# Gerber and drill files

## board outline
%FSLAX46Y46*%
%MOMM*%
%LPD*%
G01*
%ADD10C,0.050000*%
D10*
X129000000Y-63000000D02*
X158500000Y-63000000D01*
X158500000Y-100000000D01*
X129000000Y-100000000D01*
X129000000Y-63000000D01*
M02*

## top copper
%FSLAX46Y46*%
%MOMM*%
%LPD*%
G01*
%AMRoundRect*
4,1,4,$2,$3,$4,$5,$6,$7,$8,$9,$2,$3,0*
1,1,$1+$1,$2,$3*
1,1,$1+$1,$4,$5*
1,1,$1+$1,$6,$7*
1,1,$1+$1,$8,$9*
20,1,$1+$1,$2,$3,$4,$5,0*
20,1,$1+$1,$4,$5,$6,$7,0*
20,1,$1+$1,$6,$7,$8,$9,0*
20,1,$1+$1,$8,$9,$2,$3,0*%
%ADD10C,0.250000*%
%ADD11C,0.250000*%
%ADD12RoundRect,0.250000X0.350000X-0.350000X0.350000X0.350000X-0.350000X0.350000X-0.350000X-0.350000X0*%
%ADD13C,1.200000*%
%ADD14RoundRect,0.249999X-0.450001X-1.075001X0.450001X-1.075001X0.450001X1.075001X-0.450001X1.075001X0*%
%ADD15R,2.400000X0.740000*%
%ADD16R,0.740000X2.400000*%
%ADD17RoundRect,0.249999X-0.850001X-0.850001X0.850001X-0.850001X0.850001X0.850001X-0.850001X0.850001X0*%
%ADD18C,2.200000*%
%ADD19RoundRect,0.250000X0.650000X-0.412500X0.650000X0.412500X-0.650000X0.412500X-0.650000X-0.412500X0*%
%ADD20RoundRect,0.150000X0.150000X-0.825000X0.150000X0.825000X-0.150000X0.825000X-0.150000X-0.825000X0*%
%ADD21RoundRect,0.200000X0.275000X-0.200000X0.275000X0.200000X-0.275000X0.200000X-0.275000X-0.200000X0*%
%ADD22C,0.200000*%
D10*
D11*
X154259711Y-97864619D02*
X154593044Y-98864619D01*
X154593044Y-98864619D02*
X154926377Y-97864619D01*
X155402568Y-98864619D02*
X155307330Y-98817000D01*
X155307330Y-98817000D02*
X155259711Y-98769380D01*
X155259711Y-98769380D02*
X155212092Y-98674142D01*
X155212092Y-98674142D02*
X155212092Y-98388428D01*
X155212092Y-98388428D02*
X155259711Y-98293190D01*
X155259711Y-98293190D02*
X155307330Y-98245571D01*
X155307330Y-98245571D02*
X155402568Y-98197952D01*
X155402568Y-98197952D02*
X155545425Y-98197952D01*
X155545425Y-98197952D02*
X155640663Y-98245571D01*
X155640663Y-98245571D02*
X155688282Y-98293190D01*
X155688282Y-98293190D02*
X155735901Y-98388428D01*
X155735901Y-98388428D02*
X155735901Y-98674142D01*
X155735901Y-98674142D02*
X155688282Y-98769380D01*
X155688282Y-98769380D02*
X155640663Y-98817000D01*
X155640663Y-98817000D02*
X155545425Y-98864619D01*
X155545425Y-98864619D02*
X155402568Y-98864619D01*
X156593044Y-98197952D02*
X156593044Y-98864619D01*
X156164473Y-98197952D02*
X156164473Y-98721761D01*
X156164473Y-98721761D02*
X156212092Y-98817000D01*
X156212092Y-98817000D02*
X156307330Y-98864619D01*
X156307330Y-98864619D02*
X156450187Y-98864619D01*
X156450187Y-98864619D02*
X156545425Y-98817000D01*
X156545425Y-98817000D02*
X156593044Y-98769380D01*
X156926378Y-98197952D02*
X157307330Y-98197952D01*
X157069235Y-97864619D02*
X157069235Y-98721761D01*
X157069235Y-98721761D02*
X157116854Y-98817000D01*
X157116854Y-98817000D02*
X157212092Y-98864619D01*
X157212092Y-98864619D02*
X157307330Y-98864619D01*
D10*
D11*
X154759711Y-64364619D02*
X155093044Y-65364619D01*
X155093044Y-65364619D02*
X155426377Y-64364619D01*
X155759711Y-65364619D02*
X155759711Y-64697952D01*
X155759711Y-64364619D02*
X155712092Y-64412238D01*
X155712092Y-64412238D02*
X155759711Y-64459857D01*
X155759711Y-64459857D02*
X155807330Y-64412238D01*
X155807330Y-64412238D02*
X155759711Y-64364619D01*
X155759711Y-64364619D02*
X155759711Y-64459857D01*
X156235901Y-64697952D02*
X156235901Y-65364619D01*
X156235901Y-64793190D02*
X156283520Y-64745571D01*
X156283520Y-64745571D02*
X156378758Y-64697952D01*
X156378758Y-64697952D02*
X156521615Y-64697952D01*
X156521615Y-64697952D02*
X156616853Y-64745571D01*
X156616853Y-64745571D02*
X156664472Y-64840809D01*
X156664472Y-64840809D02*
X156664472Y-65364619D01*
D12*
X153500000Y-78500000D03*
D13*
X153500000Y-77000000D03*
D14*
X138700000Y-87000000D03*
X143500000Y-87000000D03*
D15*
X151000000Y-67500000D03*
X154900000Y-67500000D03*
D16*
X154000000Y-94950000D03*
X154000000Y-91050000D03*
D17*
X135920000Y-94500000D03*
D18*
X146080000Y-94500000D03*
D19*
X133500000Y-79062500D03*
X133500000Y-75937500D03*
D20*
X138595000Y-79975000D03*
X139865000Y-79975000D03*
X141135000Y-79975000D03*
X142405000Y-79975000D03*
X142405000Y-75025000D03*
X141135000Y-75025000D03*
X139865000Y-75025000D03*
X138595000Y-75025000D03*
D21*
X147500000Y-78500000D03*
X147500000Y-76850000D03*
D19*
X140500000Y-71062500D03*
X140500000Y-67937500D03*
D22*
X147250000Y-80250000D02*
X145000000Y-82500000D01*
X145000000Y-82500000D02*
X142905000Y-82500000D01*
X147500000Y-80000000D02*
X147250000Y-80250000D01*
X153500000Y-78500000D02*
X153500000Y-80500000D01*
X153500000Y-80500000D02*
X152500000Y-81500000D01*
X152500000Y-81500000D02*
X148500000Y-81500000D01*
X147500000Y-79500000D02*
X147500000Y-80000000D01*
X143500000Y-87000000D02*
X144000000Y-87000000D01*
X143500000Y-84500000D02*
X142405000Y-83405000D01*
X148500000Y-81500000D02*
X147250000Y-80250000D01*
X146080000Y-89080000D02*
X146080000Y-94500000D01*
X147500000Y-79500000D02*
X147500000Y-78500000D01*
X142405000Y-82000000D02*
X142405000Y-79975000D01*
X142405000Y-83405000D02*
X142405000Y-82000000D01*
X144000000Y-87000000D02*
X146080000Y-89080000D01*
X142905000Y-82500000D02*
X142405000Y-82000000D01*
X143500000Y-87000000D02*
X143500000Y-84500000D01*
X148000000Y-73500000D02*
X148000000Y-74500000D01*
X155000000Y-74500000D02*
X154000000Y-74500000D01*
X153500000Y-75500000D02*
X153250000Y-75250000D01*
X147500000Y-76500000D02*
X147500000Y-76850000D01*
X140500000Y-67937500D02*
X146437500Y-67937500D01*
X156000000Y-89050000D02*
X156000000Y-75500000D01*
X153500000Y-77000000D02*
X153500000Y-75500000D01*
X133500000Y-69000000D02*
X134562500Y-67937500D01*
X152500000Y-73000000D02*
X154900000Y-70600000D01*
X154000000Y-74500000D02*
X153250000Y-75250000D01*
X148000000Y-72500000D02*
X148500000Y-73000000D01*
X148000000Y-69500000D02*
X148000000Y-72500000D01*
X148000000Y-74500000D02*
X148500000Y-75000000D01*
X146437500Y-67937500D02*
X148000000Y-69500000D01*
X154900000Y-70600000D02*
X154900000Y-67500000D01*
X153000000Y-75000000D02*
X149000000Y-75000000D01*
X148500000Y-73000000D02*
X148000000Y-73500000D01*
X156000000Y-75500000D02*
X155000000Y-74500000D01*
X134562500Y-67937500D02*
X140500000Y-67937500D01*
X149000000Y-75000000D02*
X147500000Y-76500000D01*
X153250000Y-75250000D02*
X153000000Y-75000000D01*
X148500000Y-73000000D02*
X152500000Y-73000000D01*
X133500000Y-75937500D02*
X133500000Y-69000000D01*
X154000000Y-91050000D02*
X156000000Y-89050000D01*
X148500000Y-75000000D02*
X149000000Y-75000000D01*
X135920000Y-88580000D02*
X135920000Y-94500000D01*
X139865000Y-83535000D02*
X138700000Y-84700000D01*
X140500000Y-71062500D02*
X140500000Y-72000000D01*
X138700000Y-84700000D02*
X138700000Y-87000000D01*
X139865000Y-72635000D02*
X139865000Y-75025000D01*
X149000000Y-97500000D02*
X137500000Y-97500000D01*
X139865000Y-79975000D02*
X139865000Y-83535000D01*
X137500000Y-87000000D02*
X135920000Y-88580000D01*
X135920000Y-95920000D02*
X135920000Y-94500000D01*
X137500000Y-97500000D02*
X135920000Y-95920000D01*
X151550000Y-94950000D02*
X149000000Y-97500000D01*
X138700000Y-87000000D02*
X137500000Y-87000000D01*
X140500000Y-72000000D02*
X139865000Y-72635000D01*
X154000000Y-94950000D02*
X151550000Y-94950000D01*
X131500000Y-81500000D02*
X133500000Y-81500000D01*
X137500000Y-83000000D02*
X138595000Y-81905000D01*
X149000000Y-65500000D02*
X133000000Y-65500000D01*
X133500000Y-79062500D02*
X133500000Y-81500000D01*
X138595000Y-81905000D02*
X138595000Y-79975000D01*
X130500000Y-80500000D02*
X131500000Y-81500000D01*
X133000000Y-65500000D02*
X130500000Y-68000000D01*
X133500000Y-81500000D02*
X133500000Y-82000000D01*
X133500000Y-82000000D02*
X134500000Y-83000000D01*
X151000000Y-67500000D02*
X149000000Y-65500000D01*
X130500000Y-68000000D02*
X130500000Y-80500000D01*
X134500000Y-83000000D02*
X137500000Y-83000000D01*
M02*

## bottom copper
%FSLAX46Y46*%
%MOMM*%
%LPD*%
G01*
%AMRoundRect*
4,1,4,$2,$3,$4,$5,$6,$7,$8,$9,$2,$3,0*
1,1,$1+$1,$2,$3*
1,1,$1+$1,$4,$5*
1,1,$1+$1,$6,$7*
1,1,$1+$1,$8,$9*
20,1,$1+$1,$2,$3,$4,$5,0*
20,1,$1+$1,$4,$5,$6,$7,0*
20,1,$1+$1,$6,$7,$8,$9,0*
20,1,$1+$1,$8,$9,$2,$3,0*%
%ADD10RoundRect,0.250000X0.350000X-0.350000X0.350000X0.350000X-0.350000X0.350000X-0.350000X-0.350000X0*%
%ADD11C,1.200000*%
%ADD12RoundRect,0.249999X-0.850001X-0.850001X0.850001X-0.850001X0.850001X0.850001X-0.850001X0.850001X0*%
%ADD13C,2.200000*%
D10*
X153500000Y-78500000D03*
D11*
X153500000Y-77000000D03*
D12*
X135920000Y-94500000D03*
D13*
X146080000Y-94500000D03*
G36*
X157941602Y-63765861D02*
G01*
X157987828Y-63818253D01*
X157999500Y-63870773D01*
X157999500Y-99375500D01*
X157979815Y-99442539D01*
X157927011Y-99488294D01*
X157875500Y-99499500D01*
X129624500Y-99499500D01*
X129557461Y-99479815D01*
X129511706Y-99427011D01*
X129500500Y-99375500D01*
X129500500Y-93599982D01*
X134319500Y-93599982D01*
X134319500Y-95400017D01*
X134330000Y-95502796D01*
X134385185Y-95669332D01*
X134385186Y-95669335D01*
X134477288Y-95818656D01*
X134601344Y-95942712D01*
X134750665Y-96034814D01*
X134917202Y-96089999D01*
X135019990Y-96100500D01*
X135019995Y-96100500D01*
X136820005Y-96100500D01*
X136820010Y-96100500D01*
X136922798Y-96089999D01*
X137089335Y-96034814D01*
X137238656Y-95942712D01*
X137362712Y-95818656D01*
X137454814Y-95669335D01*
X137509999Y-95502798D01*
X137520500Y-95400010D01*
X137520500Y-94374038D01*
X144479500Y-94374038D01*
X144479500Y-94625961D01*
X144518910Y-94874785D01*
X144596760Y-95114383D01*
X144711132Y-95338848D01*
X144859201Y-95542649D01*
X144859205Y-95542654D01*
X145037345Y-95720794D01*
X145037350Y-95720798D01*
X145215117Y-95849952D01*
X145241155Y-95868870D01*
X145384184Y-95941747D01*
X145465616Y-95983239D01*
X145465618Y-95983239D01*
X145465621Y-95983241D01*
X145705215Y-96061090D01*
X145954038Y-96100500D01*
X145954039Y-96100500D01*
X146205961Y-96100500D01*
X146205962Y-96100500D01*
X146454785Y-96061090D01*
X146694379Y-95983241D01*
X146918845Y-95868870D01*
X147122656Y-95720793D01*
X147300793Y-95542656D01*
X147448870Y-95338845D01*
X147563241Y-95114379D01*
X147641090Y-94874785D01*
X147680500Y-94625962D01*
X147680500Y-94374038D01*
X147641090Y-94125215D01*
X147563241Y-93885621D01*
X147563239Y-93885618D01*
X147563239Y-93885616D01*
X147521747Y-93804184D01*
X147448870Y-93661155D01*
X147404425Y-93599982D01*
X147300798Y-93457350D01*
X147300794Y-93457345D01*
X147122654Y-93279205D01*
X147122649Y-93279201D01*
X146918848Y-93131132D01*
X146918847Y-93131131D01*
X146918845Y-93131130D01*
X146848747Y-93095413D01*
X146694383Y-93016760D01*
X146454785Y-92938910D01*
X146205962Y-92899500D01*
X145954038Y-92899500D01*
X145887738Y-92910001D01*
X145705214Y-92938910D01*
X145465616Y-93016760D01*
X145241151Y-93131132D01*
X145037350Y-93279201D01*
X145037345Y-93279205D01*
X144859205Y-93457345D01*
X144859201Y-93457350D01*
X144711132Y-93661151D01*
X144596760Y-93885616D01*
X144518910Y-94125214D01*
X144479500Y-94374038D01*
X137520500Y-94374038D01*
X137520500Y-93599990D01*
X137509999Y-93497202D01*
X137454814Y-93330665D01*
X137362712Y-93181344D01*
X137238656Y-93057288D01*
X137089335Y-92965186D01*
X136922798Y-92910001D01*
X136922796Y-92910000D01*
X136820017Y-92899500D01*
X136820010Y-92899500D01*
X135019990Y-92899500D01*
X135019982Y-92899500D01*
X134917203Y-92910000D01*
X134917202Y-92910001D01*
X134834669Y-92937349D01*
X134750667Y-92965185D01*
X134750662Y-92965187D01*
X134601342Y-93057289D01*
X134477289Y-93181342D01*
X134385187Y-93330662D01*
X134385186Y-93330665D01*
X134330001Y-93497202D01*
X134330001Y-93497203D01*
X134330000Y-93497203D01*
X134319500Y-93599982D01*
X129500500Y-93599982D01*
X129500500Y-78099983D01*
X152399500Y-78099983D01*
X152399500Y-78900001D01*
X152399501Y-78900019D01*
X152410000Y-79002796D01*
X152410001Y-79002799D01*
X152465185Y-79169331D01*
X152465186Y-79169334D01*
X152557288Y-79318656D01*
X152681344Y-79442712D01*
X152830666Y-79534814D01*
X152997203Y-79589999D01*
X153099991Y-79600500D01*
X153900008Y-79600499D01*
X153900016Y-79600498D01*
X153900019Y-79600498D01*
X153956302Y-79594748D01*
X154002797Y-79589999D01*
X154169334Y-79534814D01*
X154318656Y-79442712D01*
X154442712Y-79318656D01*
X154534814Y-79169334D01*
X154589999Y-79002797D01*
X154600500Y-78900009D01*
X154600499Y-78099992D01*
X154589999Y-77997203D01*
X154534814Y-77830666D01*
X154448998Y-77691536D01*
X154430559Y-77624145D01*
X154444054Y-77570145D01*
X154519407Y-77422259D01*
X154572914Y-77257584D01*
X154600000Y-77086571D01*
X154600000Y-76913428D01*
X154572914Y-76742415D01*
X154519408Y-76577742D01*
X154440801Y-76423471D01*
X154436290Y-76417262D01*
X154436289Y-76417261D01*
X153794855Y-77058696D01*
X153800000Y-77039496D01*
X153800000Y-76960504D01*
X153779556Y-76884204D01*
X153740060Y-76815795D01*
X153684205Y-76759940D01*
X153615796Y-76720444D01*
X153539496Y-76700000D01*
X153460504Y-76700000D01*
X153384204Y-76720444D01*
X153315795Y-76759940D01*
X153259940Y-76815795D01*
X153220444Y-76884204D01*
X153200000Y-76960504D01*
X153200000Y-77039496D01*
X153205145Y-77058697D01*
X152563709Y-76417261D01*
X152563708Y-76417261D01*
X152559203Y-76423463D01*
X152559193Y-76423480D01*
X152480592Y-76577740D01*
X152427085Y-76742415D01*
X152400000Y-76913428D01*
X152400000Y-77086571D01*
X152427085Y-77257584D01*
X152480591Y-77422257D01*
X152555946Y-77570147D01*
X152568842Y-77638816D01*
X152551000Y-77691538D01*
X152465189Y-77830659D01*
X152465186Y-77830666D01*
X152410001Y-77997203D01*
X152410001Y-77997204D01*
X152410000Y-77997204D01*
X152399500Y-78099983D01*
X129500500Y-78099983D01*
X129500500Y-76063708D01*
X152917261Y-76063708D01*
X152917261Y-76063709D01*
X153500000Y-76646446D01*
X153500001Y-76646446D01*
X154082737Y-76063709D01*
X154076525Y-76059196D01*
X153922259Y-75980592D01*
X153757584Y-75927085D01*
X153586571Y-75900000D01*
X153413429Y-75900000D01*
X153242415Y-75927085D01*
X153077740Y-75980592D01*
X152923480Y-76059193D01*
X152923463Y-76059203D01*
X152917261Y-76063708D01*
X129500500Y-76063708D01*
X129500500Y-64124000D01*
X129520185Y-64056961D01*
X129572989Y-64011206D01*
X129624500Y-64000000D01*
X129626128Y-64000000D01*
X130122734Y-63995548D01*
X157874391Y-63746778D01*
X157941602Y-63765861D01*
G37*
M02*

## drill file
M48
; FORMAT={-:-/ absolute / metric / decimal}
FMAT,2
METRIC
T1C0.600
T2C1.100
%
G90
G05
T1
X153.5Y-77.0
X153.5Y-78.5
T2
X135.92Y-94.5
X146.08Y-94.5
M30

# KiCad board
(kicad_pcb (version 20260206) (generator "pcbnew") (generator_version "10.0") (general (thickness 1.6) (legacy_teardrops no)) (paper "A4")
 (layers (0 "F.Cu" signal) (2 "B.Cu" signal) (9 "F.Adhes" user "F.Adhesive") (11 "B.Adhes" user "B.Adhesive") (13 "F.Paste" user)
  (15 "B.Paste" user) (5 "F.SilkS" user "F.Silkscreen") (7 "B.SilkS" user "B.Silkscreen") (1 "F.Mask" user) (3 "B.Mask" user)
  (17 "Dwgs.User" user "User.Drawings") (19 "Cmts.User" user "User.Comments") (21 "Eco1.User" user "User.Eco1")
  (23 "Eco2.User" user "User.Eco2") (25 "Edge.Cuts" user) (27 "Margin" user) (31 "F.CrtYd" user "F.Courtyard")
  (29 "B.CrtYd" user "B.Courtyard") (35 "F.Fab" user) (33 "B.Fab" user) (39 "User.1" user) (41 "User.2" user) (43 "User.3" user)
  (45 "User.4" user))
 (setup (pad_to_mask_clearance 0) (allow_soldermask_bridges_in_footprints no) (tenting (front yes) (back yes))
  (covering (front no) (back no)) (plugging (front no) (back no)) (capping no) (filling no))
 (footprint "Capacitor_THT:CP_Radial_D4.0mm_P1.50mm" (layer "F.Cu") (at 153.5 78.5 90)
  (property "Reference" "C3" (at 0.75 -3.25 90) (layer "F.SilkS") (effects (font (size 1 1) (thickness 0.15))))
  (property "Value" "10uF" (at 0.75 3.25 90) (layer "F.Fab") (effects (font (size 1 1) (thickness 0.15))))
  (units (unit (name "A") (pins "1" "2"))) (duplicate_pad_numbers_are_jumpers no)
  (pad "1" thru_hole roundrect (at 0 0 90) (size 1.2 1.2) (drill 0.6) (layers "*.Cu" "*.Mask") (remove_unused_layers no)
   (roundrect_rratio 0.208333) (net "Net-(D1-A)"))
  (pad "2" thru_hole circle (at 1.5 0 90) (size 1.2 1.2) (drill 0.6) (layers "*.Cu" "*.Mask") (remove_unused_layers no) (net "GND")))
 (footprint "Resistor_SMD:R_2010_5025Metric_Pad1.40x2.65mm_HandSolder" (layer "F.Cu") (at 141.1 87)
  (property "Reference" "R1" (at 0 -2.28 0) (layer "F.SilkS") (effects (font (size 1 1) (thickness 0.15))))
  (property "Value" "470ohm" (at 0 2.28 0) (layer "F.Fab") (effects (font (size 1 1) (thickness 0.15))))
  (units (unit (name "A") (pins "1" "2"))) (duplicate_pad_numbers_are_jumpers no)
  (pad "1" smd roundrect (at -2.4 0) (size 1.4 2.65) (layers "F.Cu" "F.Mask" "F.Paste") (roundrect_rratio 0.178571) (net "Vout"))
  (pad "2" smd roundrect (at 2.4 0) (size 1.4 2.65) (layers "F.Cu" "F.Mask" "F.Paste") (roundrect_rratio 0.178571) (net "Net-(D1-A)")))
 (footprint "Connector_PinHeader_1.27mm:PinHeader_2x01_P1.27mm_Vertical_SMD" (layer "F.Cu") (at 152.95 67.5)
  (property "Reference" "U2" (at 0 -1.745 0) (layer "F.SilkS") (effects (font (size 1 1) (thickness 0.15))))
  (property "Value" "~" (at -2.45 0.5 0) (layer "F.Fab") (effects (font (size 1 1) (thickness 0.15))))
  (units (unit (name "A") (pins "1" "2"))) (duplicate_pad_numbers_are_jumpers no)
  (pad "1" smd rect (at -1.95 0) (size 2.4 0.74) (layers "F.Cu" "F.Mask" "F.Paste") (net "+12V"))
  (pad "2" smd rect (at 1.95 0) (size 2.4 0.74) (layers "F.Cu" "F.Mask" "F.Paste") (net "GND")))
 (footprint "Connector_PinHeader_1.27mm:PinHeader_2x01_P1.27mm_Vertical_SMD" (layer "F.Cu") (at 154 93 90)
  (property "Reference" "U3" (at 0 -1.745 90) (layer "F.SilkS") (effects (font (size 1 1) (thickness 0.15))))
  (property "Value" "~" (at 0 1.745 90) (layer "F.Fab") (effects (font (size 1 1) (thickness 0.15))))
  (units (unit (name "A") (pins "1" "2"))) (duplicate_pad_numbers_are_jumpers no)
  (pad "1" smd rect (at -1.95 0 90) (size 2.4 0.74) (layers "F.Cu" "F.Mask" "F.Paste") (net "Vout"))
  (pad "2" smd rect (at 1.95 0 90) (size 2.4 0.74) (layers "F.Cu" "F.Mask" "F.Paste") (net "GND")))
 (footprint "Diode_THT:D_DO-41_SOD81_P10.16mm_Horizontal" (layer "F.Cu") (at 135.92 94.5)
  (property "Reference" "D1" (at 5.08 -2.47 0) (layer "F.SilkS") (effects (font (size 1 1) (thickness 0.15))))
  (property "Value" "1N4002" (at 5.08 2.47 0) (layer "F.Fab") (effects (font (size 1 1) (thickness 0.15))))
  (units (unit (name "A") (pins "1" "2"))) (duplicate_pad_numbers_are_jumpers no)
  (pad "1" thru_hole roundrect (at 0 0) (size 2.2 2.2) (drill 1.1) (layers "*.Cu" "*.Mask") (remove_unused_layers no)
   (roundrect_rratio 0.113636) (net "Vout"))
  (pad "2" thru_hole circle (at 10.16 0) (size 2.2 2.2) (drill 1.1) (layers "*.Cu" "*.Mask") (remove_unused_layers no) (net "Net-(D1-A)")))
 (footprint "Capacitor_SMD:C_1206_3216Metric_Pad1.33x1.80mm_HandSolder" (layer "F.Cu") (at 133.5 77.5 90)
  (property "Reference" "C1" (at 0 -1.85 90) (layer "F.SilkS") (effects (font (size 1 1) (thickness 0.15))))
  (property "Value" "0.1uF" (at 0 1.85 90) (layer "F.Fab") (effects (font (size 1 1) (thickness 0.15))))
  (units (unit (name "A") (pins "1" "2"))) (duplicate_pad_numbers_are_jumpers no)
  (pad "1" smd roundrect (at -1.5625 0 90) (size 1.325 1.8) (layers "F.Cu" "F.Mask" "F.Paste") (roundrect_rratio 0.188679) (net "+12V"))
  (pad "2" smd roundrect (at 1.5625 0 90) (size 1.325 1.8) (layers "F.Cu" "F.Mask" "F.Paste") (roundrect_rratio 0.188679) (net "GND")))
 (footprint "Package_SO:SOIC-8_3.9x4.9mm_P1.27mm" (layer "F.Cu") (at 140.5 77.5 90)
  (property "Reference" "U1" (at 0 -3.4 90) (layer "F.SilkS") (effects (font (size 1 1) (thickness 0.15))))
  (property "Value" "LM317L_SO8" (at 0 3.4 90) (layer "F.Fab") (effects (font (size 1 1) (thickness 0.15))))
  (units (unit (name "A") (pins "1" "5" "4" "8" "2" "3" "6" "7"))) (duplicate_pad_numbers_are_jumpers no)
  (pad "1" smd roundrect (at -2.475 -1.905 90) (size 1.95 0.6) (layers "F.Cu" "F.Mask" "F.Paste") (roundrect_rratio 0.25) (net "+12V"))
  (pad "2" smd roundrect (at -2.475 -0.635 90) (size 1.95 0.6) (layers "F.Cu" "F.Mask" "F.Paste") (roundrect_rratio 0.25) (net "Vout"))
  (pad "3" smd roundrect (at -2.475 0.635 90) (size 1.95 0.6) (layers "F.Cu" "F.Mask" "F.Paste") (roundrect_rratio 0.25) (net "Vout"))
  (pad "4" smd roundrect (at -2.475 1.905 90) (size 1.95 0.6) (layers "F.Cu" "F.Mask" "F.Paste") (roundrect_rratio 0.25) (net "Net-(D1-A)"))
  (pad "5" smd roundrect (at 2.475 1.905 90) (size 1.95 0.6) (layers "F.Cu" "F.Mask" "F.Paste") (roundrect_rratio 0.25)
   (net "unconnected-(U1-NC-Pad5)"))
  (pad "6" smd roundrect (at 2.475 0.635 90) (size 1.95 0.6) (layers "F.Cu" "F.Mask" "F.Paste") (roundrect_rratio 0.25) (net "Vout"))
  (pad "7" smd roundrect (at 2.475 -0.635 90) (size 1.95 0.6) (layers "F.Cu" "F.Mask" "F.Paste") (roundrect_rratio 0.25) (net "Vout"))
  (pad "8" smd roundrect (at 2.475 -1.905 90) (size 1.95 0.6) (layers "F.Cu" "F.Mask" "F.Paste") (roundrect_rratio 0.25)
   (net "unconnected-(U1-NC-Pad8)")))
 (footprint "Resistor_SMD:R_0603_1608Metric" (layer "F.Cu") (at 147.5 77.675 90)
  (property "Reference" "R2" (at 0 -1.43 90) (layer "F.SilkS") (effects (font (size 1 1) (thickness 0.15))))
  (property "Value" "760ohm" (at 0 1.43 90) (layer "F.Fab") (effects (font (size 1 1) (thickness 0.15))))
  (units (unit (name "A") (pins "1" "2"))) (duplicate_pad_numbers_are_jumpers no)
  (pad "1" smd roundrect (at -0.825 0 90) (size 0.8 0.95) (layers "F.Cu" "F.Mask" "F.Paste") (roundrect_rratio 0.25) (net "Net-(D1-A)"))
  (pad "2" smd roundrect (at 0.825 0 90) (size 0.8 0.95) (layers "F.Cu" "F.Mask" "F.Paste") (roundrect_rratio 0.25) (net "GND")))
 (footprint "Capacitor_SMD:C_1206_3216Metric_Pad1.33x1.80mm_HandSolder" (layer "F.Cu") (at 140.5 69.5 90)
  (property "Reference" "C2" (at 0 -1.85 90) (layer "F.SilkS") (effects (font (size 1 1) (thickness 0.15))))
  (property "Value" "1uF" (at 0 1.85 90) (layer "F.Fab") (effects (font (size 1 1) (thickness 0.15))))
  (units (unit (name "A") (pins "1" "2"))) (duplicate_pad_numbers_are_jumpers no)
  (pad "1" smd roundrect (at -1.5625 0 90) (size 1.325 1.8) (layers "F.Cu" "F.Mask" "F.Paste") (roundrect_rratio 0.188679) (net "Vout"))
  (pad "2" smd roundrect (at 1.5625 0 90) (size 1.325 1.8) (layers "F.Cu" "F.Mask" "F.Paste") (roundrect_rratio 0.188679) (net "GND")))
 (gr_rect (start 129 63) (end 158.5 100) (stroke (width 0.05) (type default)) (fill no) (layer "Edge.Cuts"))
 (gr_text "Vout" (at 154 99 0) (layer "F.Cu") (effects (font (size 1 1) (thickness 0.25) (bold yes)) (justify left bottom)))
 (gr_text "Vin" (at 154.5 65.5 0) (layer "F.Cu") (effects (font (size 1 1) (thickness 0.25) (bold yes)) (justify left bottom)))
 (segment (start 147.25 80.25) (end 145 82.5) (width 0.2) (layer "F.Cu") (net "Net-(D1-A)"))
 (segment (start 145 82.5) (end 142.905 82.5) (width 0.2) (layer "F.Cu") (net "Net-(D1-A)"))
 (segment (start 147.5 80) (end 147.25 80.25) (width 0.2) (layer "F.Cu") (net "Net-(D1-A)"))
 (segment (start 153.5 78.5) (end 153.5 80.5) (width 0.2) (layer "F.Cu") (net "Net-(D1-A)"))
 (segment (start 153.5 80.5) (end 152.5 81.5) (width 0.2) (layer "F.Cu") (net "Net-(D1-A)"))
 (segment (start 152.5 81.5) (end 148.5 81.5) (width 0.2) (layer "F.Cu") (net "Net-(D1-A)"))
 (segment (start 147.5 79.5) (end 147.5 80) (width 0.2) (layer "F.Cu") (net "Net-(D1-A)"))
 (segment (start 143.5 87) (end 144 87) (width 0.2) (layer "F.Cu") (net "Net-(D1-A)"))
 (segment (start 143.5 84.5) (end 142.405 83.405) (width 0.2) (layer "F.Cu") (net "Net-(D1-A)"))
 (segment (start 148.5 81.5) (end 147.25 80.25) (width 0.2) (layer "F.Cu") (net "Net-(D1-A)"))
 (segment (start 146.08 89.08) (end 146.08 94.5) (width 0.2) (layer "F.Cu") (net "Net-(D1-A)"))
 (segment (start 147.5 79.5) (end 147.5 78.5) (width 0.2) (layer "F.Cu") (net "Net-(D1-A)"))
 (segment (start 142.405 82) (end 142.405 79.975) (width 0.2) (layer "F.Cu") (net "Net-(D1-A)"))
 (segment (start 142.405 83.405) (end 142.405 82) (width 0.2) (layer "F.Cu") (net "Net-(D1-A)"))
 (segment (start 144 87) (end 146.08 89.08) (width 0.2) (layer "F.Cu") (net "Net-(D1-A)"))
 (segment (start 142.905 82.5) (end 142.405 82) (width 0.2) (layer "F.Cu") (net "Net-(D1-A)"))
 (segment (start 143.5 87) (end 143.5 84.5) (width 0.2) (layer "F.Cu") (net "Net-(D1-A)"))
 (segment (start 148 73.5) (end 148 74.5) (width 0.2) (layer "F.Cu") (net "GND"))
 (segment (start 155 74.5) (end 154 74.5) (width 0.2) (layer "F.Cu") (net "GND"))
 (segment (start 153.5 75.5) (end 153.25 75.25) (width 0.2) (layer "F.Cu") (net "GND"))
 (segment (start 147.5 76.5) (end 147.5 76.85) (width 0.2) (layer "F.Cu") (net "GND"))
 (segment (start 140.5 67.9375) (end 146.4375 67.9375) (width 0.2) (layer "F.Cu") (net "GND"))
 (segment (start 156 89.05) (end 156 75.5) (width 0.2) (layer "F.Cu") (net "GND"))
 (segment (start 153.5 77) (end 153.5 75.5) (width 0.2) (layer "F.Cu") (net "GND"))
 (segment (start 133.5 69) (end 134.5625 67.9375) (width 0.2) (layer "F.Cu") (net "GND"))
 (segment (start 152.5 73) (end 154.9 70.6) (width 0.2) (layer "F.Cu") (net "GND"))
 (segment (start 154 74.5) (end 153.25 75.25) (width 0.2) (layer "F.Cu") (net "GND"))
 (segment (start 148 72.5) (end 148.5 73) (width 0.2) (layer "F.Cu") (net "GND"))
 (segment (start 148 69.5) (end 148 72.5) (width 0.2) (layer "F.Cu") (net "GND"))
 (segment (start 148 74.5) (end 148.5 75) (width 0.2) (layer "F.Cu") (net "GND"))
 (segment (start 146.4375 67.9375) (end 148 69.5) (width 0.2) (layer "F.Cu") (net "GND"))
 (segment (start 154.9 70.6) (end 154.9 67.5) (width 0.2) (layer "F.Cu") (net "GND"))
 (segment (start 153 75) (end 149 75) (width 0.2) (layer "F.Cu") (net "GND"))
 (segment (start 148.5 73) (end 148 73.5) (width 0.2) (layer "F.Cu") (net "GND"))
 (segment (start 156 75.5) (end 155 74.5) (width 0.2) (layer "F.Cu") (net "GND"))
 (segment (start 134.5625 67.9375) (end 140.5 67.9375) (width 0.2) (layer "F.Cu") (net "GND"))
 (segment (start 149 75) (end 147.5 76.5) (width 0.2) (layer "F.Cu") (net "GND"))
 (segment (start 153.25 75.25) (end 153 75) (width 0.2) (layer "F.Cu") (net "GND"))
 (segment (start 148.5 73) (end 152.5 73) (width 0.2) (layer "F.Cu") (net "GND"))
 (segment (start 133.5 75.9375) (end 133.5 69) (width 0.2) (layer "F.Cu") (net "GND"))
 (segment (start 154 91.05) (end 156 89.05) (width 0.2) (layer "F.Cu") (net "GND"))
 (segment (start 148.5 75) (end 149 75) (width 0.2) (layer "F.Cu") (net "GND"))
 (segment (start 135.92 88.58) (end 135.92 94.5) (width 0.2) (layer "F.Cu") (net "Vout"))
 (segment (start 139.865 83.535) (end 138.7 84.7) (width 0.2) (layer "F.Cu") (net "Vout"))
 (segment (start 140.5 71.0625) (end 140.5 72) (width 0.2) (layer "F.Cu") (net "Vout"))
 (segment (start 138.7 84.7) (end 138.7 87) (width 0.2) (layer "F.Cu") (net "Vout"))
 (segment (start 139.865 72.635) (end 139.865 75.025) (width 0.2) (layer "F.Cu") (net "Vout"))
 (segment (start 149 97.5) (end 137.5 97.5) (width 0.2) (layer "F.Cu") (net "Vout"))
 (segment (start 139.865 79.975) (end 139.865 83.535) (width 0.2) (layer "F.Cu") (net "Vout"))
 (segment (start 137.5 87) (end 135.92 88.58) (width 0.2) (layer "F.Cu") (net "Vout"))
 (segment (start 135.92 95.92) (end 135.92 94.5) (width 0.2) (layer "F.Cu") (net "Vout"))
 (segment (start 137.5 97.5) (end 135.92 95.92) (width 0.2) (layer "F.Cu") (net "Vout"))
 (segment (start 151.55 94.95) (end 149 97.5) (width 0.2) (layer "F.Cu") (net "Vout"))
 (segment (start 138.7 87) (end 137.5 87) (width 0.2) (layer "F.Cu") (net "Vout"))
 (segment (start 140.5 72) (end 139.865 72.635) (width 0.2) (layer "F.Cu") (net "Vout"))
 (segment (start 154 94.95) (end 151.55 94.95) (width 0.2) (layer "F.Cu") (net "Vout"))
 (segment (start 131.5 81.5) (end 133.5 81.5) (width 0.2) (layer "F.Cu") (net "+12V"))
 (segment (start 137.5 83) (end 138.595 81.905) (width 0.2) (layer "F.Cu") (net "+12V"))
 (segment (start 149 65.5) (end 133 65.5) (width 0.2) (layer "F.Cu") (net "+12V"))
 (segment (start 133.5 79.0625) (end 133.5 81.5) (width 0.2) (layer "F.Cu") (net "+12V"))
 (segment (start 138.595 81.905) (end 138.595 79.975) (width 0.2) (layer "F.Cu") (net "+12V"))
 (segment (start 130.5 80.5) (end 131.5 81.5) (width 0.2) (layer "F.Cu") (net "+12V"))
 (segment (start 133 65.5) (end 130.5 68) (width 0.2) (layer "F.Cu") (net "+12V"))
 (segment (start 133.5 81.5) (end 133.5 82) (width 0.2) (layer "F.Cu") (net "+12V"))
 (segment (start 133.5 82) (end 134.5 83) (width 0.2) (layer "F.Cu") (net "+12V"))
 (segment (start 151 67.5) (end 149 65.5) (width 0.2) (layer "F.Cu") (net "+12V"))
 (segment (start 130.5 68) (end 130.5 80.5) (width 0.2) (layer "F.Cu") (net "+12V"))
 (segment (start 134.5 83) (end 137.5 83) (width 0.2) (layer "F.Cu") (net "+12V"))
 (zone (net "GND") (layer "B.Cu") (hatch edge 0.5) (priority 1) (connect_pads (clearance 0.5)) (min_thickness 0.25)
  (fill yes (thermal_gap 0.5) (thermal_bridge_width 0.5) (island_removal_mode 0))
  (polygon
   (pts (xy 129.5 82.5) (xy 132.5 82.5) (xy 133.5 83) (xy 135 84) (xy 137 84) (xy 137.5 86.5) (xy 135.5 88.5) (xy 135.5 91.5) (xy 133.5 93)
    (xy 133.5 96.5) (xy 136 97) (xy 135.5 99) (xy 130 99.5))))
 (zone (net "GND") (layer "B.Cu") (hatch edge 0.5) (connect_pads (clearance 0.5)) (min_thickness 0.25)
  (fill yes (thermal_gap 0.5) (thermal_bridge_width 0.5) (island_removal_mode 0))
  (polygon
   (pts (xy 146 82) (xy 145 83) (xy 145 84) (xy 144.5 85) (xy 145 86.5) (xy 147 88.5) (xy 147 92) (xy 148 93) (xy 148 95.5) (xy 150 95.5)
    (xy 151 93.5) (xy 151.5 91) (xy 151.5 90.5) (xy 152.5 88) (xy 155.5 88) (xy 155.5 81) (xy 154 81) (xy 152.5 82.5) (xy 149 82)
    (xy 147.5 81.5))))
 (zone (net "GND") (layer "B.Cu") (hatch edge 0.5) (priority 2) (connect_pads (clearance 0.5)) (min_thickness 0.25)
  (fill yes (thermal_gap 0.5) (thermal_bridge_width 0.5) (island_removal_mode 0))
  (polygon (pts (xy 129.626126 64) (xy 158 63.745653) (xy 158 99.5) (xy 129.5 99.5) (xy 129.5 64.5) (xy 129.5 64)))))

